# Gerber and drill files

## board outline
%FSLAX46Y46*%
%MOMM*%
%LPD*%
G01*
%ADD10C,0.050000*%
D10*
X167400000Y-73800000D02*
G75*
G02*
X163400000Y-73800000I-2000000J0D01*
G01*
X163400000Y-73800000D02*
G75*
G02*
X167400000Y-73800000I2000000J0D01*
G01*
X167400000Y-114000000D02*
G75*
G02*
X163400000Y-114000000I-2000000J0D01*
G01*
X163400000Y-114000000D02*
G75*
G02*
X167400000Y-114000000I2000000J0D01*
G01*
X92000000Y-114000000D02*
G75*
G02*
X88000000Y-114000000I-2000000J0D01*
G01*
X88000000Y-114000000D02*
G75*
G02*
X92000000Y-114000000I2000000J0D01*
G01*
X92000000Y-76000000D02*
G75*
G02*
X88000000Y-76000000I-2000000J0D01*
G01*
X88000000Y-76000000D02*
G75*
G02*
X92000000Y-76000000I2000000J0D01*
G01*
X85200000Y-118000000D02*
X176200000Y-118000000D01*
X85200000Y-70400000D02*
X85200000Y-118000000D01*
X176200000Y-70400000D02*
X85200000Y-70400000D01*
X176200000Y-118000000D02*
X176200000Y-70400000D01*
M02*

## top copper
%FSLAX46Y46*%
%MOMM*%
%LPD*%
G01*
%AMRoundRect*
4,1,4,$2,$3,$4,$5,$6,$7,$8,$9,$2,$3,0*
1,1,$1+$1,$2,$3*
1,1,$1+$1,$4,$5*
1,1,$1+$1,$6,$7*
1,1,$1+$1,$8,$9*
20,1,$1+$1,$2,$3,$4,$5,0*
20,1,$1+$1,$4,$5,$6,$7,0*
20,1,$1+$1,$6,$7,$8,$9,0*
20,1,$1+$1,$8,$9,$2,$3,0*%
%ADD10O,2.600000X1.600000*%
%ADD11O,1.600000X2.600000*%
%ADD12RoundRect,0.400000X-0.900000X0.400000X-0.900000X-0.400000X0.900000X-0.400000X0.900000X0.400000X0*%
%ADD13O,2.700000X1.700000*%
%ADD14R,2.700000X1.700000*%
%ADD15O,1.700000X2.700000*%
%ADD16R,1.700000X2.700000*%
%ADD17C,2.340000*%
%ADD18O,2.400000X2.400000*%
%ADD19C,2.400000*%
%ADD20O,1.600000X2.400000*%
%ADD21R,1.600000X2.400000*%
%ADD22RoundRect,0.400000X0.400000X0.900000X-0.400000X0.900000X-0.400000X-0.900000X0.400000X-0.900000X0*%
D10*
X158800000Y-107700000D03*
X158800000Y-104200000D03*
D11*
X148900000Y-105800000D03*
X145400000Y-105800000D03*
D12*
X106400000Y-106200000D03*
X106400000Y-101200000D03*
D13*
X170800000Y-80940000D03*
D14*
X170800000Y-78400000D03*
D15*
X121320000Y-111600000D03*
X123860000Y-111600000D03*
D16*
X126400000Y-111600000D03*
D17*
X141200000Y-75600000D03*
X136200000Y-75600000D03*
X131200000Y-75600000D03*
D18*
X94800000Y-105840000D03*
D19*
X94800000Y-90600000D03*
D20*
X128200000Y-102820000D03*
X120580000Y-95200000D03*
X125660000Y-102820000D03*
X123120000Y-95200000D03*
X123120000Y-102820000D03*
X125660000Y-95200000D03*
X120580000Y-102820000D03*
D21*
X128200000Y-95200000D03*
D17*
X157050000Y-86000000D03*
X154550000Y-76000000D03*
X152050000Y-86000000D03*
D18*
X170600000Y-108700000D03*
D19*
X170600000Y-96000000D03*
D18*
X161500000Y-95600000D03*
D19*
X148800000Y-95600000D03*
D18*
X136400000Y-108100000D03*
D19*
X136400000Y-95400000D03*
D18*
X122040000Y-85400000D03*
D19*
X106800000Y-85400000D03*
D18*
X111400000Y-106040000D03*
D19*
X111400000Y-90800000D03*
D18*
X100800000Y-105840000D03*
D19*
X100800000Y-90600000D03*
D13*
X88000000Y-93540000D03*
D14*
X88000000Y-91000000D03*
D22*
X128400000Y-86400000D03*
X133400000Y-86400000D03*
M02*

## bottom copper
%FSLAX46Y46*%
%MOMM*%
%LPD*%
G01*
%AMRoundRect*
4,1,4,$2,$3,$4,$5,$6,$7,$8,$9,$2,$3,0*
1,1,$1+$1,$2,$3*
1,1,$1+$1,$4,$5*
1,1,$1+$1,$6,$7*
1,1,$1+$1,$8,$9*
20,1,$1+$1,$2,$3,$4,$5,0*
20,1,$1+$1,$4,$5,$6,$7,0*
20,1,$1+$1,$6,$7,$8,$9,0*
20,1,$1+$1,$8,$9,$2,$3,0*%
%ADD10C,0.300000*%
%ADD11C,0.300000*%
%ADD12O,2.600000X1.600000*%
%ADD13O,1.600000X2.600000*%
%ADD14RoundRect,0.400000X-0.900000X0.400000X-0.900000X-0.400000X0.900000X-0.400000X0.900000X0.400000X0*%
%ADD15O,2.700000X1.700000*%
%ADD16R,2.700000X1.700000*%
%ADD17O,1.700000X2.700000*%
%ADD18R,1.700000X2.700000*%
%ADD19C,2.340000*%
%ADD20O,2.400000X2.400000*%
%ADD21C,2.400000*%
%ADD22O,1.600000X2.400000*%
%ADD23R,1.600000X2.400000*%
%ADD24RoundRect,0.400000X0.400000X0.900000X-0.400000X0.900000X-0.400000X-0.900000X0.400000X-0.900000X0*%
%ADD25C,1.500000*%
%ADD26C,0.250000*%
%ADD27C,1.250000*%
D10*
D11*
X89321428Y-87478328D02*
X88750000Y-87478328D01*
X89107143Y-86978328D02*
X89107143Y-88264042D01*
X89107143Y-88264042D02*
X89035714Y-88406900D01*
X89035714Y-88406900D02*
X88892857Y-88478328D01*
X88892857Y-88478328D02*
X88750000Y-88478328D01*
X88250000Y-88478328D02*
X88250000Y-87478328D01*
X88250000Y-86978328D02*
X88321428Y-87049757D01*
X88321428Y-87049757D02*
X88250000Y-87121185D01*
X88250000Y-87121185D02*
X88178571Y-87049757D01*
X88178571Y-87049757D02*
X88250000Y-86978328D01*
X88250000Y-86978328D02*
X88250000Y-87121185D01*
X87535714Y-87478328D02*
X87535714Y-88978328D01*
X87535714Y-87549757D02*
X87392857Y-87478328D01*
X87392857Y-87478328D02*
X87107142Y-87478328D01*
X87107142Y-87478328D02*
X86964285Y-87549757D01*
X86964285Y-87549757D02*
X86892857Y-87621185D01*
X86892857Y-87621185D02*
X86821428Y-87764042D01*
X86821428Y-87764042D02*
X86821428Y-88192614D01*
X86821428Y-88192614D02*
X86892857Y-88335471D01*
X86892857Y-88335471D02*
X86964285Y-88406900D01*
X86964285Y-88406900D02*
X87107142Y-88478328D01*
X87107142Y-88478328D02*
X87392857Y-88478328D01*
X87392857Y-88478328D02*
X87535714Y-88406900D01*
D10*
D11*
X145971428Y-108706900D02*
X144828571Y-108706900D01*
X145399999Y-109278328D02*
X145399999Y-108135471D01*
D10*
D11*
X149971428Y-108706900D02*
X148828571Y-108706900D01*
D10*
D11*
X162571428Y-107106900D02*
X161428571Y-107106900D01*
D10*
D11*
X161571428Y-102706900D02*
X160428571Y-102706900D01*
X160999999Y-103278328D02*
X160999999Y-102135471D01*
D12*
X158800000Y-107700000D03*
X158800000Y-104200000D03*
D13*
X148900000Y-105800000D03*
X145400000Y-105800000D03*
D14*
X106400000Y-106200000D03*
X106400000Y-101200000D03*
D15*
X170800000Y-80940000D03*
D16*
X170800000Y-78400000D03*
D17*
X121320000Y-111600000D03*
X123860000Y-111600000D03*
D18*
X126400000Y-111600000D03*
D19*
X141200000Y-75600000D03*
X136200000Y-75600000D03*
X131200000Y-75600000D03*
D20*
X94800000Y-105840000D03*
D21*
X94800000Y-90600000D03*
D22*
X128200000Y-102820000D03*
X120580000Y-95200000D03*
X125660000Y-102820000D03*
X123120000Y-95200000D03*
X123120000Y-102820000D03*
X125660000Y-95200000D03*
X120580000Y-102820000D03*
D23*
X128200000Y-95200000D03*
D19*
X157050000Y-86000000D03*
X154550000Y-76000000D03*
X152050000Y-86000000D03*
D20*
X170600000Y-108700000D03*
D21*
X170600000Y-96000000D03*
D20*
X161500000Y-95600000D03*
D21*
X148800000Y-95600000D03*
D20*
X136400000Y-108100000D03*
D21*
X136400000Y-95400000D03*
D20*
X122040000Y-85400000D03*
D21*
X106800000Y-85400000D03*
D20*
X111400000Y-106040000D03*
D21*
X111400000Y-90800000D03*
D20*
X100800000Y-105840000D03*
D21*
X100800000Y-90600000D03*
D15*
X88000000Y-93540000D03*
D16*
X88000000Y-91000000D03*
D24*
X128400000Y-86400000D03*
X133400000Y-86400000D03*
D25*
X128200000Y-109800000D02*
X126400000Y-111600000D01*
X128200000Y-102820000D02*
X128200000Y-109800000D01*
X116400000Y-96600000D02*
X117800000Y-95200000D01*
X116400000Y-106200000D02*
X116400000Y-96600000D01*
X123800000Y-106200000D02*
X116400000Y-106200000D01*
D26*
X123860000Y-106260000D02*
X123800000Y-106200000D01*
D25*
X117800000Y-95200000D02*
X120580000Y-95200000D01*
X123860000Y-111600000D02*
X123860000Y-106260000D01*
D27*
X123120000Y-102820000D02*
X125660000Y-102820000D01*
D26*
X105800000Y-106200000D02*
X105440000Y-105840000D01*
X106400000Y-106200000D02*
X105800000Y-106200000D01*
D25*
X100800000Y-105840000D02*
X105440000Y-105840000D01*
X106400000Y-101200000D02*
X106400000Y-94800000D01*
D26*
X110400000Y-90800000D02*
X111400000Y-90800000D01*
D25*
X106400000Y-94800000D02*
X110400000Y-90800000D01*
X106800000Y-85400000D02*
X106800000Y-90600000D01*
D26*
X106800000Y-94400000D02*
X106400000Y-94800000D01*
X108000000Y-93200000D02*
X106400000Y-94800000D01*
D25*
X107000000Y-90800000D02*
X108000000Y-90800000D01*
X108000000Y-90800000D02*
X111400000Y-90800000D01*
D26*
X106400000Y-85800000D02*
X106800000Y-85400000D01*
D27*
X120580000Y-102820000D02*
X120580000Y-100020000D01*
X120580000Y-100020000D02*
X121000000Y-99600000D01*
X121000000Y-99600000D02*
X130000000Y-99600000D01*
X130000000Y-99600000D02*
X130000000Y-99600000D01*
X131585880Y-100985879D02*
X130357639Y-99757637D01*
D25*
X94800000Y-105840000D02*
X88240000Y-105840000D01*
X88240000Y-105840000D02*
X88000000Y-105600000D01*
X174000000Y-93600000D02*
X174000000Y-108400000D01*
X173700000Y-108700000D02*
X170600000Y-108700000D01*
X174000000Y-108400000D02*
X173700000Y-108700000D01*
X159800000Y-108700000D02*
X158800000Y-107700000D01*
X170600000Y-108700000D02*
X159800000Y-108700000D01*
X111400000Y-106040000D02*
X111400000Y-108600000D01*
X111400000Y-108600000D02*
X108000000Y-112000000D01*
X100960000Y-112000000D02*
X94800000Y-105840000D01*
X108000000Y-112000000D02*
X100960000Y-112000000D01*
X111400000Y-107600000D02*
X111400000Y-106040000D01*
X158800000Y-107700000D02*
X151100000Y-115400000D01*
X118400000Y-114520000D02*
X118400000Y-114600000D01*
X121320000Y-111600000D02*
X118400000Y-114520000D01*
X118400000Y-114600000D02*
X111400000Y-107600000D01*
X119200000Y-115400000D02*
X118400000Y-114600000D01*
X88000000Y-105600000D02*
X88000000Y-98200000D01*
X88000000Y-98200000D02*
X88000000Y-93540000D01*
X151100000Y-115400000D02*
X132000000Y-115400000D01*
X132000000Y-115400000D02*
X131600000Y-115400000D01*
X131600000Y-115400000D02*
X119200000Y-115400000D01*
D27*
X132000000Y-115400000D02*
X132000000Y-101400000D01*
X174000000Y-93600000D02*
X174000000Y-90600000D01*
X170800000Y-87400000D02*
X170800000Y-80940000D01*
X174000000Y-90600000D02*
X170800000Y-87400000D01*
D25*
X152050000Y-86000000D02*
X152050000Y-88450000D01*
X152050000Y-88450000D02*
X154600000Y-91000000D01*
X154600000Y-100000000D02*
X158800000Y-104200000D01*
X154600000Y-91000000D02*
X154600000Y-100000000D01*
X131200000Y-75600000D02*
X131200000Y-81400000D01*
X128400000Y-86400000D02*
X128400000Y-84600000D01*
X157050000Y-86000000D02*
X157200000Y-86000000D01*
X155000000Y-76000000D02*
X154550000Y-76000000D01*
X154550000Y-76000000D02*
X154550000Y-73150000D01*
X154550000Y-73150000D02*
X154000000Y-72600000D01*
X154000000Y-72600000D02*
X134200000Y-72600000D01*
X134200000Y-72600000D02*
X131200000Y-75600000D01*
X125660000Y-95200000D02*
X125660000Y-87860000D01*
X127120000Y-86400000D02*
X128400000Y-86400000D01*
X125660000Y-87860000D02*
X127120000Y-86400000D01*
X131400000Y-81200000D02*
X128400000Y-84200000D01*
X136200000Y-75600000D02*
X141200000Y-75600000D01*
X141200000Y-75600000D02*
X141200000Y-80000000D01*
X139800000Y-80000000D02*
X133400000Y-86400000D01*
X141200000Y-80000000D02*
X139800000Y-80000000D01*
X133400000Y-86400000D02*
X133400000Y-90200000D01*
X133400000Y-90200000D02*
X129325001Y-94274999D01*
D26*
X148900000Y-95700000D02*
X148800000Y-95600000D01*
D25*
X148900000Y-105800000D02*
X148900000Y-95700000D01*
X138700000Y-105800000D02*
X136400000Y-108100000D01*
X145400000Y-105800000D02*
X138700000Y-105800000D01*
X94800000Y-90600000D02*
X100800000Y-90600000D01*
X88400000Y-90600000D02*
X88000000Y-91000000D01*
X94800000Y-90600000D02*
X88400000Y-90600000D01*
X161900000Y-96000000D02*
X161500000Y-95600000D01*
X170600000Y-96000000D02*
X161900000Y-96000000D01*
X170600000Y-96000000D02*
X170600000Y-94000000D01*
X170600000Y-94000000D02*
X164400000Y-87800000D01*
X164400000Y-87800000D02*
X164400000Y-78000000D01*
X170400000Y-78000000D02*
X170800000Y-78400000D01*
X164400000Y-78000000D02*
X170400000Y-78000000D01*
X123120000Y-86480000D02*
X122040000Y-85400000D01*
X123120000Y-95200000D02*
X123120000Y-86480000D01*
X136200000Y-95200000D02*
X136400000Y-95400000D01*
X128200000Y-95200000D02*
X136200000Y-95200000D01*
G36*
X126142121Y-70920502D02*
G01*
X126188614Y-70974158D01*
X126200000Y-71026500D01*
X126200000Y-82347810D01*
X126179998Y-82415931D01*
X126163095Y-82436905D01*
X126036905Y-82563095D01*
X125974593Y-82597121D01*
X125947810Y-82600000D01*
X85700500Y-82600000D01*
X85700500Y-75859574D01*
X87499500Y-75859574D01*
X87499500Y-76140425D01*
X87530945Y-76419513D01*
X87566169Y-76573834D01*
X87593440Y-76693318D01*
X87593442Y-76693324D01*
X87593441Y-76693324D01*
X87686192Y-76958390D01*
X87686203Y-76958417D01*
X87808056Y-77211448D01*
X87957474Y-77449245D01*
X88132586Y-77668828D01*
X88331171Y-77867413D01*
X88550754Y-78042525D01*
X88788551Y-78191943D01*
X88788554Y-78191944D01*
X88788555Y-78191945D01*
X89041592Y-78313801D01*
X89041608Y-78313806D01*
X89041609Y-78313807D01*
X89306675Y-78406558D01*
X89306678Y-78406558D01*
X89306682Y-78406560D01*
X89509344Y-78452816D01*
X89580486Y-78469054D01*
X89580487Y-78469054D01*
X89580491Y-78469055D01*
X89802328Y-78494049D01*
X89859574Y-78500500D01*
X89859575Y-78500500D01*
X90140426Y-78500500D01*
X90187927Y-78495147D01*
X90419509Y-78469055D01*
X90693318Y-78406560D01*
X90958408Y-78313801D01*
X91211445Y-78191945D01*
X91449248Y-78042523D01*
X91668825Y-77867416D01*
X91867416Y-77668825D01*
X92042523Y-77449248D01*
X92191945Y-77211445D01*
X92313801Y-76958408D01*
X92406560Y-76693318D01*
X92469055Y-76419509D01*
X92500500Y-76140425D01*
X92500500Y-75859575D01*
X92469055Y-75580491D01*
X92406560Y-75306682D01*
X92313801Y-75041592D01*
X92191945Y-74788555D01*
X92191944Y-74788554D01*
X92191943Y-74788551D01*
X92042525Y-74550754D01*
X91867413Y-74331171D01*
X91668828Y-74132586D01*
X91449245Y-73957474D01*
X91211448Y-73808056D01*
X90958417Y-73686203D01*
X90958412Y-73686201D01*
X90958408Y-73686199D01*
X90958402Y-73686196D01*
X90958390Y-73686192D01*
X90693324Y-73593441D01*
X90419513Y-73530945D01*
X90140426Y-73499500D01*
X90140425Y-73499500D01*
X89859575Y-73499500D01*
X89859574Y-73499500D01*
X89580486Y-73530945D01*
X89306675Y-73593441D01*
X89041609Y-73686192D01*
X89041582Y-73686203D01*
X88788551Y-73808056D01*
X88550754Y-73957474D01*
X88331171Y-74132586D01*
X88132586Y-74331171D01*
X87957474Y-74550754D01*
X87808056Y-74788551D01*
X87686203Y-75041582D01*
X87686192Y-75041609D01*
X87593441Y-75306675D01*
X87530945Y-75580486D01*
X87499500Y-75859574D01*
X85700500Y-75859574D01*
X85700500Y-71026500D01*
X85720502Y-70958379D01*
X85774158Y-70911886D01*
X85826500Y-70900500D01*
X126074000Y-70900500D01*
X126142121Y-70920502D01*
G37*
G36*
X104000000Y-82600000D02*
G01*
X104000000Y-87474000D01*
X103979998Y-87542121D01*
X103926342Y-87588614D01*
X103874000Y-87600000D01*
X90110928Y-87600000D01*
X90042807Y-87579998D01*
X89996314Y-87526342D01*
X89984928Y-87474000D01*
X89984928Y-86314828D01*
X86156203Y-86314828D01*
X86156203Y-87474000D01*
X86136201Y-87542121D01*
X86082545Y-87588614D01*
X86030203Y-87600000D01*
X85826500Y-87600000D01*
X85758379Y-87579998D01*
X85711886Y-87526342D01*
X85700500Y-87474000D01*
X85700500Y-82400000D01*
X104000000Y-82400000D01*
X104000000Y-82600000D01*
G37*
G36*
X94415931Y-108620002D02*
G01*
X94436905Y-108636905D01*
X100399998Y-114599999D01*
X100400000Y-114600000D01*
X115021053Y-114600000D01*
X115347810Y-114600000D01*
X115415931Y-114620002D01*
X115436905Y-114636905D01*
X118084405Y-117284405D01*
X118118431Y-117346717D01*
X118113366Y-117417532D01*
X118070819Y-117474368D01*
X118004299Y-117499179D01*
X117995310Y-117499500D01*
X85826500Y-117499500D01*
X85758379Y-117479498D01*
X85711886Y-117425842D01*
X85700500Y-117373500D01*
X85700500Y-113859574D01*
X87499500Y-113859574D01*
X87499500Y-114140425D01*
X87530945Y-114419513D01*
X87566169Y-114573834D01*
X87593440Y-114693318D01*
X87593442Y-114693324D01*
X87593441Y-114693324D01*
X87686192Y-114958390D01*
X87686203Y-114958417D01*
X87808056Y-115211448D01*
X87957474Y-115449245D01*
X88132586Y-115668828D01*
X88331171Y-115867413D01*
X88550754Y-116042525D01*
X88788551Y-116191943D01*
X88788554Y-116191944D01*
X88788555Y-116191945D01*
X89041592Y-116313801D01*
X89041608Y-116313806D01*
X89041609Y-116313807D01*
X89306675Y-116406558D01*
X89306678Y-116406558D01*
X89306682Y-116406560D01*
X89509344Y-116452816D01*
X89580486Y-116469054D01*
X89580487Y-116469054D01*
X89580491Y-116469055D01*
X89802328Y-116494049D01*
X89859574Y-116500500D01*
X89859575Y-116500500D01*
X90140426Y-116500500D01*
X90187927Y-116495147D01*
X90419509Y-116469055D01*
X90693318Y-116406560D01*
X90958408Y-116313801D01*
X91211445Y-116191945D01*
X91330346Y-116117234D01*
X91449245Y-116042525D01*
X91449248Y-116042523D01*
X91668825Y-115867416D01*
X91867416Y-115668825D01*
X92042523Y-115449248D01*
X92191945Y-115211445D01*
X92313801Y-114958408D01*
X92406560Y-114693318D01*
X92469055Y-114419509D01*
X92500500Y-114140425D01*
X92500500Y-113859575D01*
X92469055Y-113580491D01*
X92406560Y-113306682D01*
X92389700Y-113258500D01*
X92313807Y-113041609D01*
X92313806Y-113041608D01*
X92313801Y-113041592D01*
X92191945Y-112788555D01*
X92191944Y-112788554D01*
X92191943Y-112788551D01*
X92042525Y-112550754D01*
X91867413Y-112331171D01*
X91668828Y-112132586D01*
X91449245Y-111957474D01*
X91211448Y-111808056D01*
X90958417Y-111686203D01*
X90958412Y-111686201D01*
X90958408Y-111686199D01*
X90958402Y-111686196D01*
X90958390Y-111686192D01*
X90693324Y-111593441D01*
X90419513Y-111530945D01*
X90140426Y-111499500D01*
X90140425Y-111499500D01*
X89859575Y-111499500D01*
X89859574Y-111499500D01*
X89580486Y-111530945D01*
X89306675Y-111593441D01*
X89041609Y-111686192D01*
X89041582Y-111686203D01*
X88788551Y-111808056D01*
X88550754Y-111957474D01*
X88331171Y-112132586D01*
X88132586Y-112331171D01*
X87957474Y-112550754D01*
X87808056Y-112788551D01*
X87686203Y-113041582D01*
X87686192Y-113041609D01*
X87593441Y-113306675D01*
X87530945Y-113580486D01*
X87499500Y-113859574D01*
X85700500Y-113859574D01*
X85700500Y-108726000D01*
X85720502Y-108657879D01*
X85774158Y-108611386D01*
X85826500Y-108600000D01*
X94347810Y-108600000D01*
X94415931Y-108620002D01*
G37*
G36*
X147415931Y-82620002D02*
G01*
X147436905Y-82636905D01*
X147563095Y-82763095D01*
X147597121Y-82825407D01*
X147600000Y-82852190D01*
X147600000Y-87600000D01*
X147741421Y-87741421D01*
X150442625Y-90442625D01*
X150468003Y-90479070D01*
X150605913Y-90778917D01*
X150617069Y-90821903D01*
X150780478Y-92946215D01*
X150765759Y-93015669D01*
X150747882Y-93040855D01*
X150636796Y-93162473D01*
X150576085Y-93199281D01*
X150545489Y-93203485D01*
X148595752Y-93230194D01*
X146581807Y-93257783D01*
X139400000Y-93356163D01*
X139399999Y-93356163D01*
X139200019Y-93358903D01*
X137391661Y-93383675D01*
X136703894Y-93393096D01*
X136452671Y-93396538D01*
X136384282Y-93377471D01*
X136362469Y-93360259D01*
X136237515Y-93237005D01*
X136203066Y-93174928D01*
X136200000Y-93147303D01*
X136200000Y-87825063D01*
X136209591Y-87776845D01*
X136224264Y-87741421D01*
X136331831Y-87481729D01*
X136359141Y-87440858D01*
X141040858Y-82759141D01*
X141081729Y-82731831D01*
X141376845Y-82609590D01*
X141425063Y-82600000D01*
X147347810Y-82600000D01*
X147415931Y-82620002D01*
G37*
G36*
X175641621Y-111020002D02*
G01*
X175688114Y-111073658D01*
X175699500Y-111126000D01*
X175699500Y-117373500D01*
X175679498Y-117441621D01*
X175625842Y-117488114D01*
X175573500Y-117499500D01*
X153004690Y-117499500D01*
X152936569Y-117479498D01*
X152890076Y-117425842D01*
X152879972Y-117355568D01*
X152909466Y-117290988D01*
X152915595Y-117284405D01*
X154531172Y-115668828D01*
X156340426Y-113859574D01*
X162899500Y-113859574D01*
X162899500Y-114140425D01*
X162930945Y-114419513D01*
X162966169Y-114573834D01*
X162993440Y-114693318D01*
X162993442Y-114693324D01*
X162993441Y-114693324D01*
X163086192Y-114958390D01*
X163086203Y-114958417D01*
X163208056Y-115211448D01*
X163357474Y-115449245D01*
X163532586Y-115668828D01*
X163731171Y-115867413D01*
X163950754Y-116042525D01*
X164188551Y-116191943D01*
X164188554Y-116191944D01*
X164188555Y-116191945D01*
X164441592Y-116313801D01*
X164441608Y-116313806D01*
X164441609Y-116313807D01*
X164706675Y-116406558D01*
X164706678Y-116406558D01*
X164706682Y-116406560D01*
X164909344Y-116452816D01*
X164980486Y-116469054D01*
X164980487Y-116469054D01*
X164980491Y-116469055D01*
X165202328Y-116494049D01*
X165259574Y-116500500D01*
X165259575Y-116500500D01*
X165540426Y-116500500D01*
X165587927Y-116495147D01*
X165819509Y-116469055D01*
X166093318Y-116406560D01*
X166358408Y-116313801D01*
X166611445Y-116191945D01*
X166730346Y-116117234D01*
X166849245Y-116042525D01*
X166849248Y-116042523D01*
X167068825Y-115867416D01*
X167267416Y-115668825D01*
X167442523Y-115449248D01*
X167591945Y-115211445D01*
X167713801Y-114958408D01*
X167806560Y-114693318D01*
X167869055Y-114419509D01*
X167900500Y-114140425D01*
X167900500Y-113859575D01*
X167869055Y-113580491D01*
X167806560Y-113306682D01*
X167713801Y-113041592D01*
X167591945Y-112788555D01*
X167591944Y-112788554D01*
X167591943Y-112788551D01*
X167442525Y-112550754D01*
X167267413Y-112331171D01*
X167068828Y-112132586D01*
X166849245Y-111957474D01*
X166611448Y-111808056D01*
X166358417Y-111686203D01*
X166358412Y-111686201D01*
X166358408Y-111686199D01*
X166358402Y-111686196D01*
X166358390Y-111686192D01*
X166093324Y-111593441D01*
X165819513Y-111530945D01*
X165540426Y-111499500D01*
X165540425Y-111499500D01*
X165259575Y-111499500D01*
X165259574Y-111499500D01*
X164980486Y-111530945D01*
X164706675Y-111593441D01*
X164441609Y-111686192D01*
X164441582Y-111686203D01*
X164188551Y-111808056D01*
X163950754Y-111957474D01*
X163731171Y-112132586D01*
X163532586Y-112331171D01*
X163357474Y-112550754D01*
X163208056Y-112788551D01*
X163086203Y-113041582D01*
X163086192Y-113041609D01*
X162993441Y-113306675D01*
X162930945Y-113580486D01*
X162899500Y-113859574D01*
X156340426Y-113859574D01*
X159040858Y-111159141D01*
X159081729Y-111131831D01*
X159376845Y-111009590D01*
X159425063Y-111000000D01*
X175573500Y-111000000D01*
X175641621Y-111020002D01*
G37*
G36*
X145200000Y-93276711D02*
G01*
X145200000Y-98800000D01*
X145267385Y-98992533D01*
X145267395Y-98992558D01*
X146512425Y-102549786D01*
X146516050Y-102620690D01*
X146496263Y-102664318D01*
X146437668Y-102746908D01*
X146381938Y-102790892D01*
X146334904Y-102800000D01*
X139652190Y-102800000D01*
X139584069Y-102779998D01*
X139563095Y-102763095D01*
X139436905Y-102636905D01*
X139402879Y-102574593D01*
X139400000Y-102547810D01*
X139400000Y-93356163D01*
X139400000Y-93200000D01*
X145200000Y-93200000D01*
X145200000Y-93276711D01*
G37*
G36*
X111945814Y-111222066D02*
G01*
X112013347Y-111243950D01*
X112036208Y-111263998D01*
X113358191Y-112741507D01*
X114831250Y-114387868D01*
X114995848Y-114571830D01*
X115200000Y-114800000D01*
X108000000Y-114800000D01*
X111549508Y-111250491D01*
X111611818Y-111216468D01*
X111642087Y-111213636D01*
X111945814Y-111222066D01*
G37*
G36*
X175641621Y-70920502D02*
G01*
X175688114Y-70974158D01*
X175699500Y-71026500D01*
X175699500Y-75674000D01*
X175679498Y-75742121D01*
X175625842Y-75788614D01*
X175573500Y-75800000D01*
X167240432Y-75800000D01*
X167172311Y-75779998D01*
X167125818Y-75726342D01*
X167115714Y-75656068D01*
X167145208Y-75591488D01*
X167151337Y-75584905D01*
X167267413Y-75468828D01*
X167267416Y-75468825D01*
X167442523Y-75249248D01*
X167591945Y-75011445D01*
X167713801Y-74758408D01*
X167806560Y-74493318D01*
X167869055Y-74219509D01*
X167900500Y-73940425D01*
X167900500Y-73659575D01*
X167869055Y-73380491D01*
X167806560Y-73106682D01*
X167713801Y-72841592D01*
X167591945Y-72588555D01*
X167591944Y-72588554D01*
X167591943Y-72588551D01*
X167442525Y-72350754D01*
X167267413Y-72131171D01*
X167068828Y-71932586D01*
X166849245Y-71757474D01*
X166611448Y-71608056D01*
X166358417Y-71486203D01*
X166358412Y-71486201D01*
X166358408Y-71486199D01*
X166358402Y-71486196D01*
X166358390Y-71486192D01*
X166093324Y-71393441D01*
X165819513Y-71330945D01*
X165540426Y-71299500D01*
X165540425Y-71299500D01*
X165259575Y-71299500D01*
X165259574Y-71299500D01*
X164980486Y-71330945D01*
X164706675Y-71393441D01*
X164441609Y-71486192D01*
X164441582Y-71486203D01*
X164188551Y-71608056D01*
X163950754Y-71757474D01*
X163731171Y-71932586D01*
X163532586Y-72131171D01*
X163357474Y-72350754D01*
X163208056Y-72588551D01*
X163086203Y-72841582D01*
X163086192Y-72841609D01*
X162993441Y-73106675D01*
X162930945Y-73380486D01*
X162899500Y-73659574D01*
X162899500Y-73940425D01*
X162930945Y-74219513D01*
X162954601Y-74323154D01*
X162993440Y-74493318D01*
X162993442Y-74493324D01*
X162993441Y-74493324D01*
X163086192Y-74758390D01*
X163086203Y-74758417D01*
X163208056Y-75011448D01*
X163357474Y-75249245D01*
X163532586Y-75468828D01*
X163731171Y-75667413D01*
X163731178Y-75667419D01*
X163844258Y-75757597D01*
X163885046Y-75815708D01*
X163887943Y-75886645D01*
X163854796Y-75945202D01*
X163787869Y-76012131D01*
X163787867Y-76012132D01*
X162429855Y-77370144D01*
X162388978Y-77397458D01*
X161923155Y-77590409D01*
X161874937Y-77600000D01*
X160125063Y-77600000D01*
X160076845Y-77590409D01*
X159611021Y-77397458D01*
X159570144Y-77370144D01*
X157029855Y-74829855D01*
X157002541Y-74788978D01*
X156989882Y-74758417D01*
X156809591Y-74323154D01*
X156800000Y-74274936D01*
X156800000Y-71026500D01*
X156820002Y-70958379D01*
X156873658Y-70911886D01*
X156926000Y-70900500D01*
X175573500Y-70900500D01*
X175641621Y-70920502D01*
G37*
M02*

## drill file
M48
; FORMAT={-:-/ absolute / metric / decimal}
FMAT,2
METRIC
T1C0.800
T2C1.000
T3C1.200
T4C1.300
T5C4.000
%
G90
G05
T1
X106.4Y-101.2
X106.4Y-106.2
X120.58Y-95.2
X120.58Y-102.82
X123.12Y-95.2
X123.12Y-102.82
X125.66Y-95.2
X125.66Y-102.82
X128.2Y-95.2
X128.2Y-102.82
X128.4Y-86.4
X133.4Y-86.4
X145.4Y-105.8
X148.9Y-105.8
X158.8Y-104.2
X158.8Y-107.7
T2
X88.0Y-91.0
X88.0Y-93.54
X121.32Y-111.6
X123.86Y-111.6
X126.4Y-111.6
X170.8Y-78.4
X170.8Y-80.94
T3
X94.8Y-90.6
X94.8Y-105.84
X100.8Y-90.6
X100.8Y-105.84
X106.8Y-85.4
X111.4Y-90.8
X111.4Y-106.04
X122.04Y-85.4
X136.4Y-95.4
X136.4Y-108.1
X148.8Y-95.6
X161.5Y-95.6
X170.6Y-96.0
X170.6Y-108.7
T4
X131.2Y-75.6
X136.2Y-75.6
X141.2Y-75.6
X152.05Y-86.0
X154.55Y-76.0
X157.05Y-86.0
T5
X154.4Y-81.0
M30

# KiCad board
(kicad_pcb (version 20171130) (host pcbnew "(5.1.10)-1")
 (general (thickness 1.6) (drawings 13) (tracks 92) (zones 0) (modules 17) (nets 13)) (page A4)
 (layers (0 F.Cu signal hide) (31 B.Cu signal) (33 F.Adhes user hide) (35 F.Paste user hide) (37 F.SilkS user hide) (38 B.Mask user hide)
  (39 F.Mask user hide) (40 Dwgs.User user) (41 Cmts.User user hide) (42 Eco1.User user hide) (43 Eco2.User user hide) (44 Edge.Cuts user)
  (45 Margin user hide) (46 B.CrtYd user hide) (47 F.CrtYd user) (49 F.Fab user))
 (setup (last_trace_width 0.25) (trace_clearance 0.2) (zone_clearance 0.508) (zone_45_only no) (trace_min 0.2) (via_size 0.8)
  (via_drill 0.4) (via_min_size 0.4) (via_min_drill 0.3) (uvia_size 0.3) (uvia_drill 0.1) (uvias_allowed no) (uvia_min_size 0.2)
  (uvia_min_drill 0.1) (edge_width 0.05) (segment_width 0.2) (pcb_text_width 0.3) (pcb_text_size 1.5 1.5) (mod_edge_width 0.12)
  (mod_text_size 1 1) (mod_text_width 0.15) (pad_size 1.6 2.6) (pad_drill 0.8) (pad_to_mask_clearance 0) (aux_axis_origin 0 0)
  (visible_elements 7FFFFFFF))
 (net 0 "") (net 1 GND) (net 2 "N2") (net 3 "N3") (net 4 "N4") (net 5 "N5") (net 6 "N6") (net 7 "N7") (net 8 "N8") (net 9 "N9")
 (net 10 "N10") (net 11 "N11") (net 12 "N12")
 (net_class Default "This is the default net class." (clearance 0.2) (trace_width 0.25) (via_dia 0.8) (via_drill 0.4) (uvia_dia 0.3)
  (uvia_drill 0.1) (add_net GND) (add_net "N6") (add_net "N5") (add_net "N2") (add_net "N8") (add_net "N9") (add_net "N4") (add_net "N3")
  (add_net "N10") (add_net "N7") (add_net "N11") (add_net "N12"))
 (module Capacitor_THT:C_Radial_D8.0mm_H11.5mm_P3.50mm (layer F.Cu) (at 158.8 104.2 270)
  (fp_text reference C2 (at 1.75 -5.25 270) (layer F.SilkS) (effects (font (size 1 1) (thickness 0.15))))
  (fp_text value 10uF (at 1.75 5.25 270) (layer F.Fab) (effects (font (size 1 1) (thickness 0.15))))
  (pad 2 thru_hole oval (at 3.5 0 270) (size 1.6 2.6) (drill 0.8) (layers *.Cu *.Mask) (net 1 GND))
  (pad 1 thru_hole oval (at 0 0 270) (size 1.6 2.6) (drill 0.8) (layers *.Cu *.Mask) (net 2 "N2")))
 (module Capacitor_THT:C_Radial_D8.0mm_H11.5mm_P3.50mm (layer F.Cu) (at 145.4 105.8)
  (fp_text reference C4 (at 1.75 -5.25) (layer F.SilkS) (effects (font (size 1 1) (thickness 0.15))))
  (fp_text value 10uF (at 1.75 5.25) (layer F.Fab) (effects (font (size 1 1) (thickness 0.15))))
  (pad 2 thru_hole oval (at 3.5 0) (size 1.6 2.6) (drill 0.8) (layers *.Cu *.Mask) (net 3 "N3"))
  (pad 1 thru_hole oval (at 0 0) (size 1.6 2.6) (drill 0.8) (layers *.Cu *.Mask) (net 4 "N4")))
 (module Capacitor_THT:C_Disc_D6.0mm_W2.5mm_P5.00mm (layer F.Cu) (at 106.4 101.2 270)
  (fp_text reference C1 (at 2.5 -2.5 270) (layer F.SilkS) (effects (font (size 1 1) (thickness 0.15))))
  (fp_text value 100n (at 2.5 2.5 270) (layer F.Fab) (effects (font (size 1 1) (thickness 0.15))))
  (pad 2 thru_hole roundrect (at 5 0 270) (size 1.6 2.6) (drill 0.8) (layers *.Cu *.Mask) (roundrect_rratio 0.25) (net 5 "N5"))
  (pad 1 thru_hole roundrect (at 0 0 270) (size 1.6 2.6) (drill 0.8) (layers *.Cu *.Mask) (roundrect_rratio 0.25) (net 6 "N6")))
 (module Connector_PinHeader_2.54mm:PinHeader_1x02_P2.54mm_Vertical (layer F.Cu) (at 170.8 78.4)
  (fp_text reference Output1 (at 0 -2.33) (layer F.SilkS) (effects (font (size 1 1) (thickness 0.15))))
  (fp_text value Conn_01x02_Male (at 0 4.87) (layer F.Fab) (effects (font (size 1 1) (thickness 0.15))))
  (pad 2 thru_hole oval (at 0 2.54) (size 2.7 1.7) (drill 1) (layers *.Cu *.Mask) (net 1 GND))
  (pad 1 thru_hole rect (at 0 0) (size 2.7 1.7) (drill 1) (layers *.Cu *.Mask) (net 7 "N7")))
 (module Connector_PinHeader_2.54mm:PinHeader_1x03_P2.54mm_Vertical (layer F.Cu) (at 126.4 111.6 270)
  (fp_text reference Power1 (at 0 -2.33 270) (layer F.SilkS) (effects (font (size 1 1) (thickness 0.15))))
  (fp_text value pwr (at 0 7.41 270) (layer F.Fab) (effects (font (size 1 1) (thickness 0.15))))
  (pad 3 thru_hole oval (at 0 5.08 270) (size 2.7 1.7) (drill 1) (layers *.Cu *.Mask) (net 1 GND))
  (pad 2 thru_hole oval (at 0 2.54 270) (size 2.7 1.7) (drill 1) (layers *.Cu *.Mask))
  (pad 1 thru_hole rect (at 0 0 270) (size 2.7 1.7) (drill 1) (layers *.Cu *.Mask)))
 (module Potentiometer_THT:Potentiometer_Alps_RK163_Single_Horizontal (layer F.Cu) (at 141.2 75.6 90)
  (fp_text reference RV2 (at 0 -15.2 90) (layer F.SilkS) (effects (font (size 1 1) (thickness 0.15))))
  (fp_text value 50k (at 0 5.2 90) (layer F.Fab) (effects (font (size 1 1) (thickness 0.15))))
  (pad 1 thru_hole circle (at 0 0 90) (size 2.34 2.34) (drill 1.3) (layers *.Cu *.Mask) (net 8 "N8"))
  (pad 2 thru_hole circle (at 0 -5 90) (size 2.34 2.34) (drill 1.3) (layers *.Cu *.Mask) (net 8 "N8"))
  (pad 3 thru_hole circle (at 0 -10 90) (size 2.34 2.34) (drill 1.3) (layers *.Cu *.Mask) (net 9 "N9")))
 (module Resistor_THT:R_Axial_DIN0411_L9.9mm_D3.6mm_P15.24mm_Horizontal (layer F.Cu) (at 94.8 90.6 270)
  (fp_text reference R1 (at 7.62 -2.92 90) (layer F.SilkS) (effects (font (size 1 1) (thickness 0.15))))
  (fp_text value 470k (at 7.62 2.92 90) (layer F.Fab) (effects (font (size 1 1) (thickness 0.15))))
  (pad 2 thru_hole oval (at 15.24 0 270) (size 2.4 2.4) (drill 1.2) (layers *.Cu *.Mask) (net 1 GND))
  (pad 1 thru_hole circle (at 0 0 270) (size 2.4 2.4) (drill 1.2) (layers *.Cu *.Mask) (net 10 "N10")))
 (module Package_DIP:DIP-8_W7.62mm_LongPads (layer F.Cu) (at 128.2 95.2 270)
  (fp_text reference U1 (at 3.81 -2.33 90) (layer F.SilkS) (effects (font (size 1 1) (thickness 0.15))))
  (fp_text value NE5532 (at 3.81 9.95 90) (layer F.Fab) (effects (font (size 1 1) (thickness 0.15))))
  (pad 8 thru_hole oval (at 7.62 0 270) (size 2.4 1.6) (drill 0.8) (layers *.Cu *.Mask))
  (pad 4 thru_hole oval (at 0 7.62 270) (size 2.4 1.6) (drill 0.8) (layers *.Cu *.Mask))
  (pad 7 thru_hole oval (at 7.62 2.54 270) (size 2.4 1.6) (drill 0.8) (layers *.Cu *.Mask))
  (pad 3 thru_hole oval (at 0 5.08 270) (size 2.4 1.6) (drill 0.8) (layers *.Cu *.Mask) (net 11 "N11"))
  (pad 6 thru_hole oval (at 7.62 5.08 270) (size 2.4 1.6) (drill 0.8) (layers *.Cu *.Mask))
  (pad 2 thru_hole oval (at 0 2.54 270) (size 2.4 1.6) (drill 0.8) (layers *.Cu *.Mask) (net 9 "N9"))
  (pad 5 thru_hole oval (at 7.62 7.62 270) (size 2.4 1.6) (drill 0.8) (layers *.Cu *.Mask) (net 1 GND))
  (pad 1 thru_hole rect (at 0 0 270) (size 2.4 1.6) (drill 0.8) (layers *.Cu *.Mask) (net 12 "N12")))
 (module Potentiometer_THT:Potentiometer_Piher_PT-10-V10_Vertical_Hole (layer F.Cu) (at 157.05 86 90)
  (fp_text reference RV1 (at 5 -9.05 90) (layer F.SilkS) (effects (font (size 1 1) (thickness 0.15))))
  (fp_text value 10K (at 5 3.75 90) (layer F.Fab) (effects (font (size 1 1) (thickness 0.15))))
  (pad "" np_thru_hole circle (at 5 -2.65 90) (size 4 4) (drill 4) (layers *.Cu *.Mask))
  (pad 1 thru_hole circle (at 0 0 90) (size 2.34 2.34) (drill 1.3) (layers *.Cu *.Mask) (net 9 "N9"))
  (pad 2 thru_hole circle (at 10 -2.5 90) (size 2.34 2.34) (drill 1.3) (layers *.Cu *.Mask) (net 9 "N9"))
  (pad 3 thru_hole circle (at 0 -5 90) (size 2.34 2.34) (drill 1.3) (layers *.Cu *.Mask) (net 2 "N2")))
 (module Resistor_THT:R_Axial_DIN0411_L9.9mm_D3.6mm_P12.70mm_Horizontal (layer F.Cu) (at 170.6 96 270)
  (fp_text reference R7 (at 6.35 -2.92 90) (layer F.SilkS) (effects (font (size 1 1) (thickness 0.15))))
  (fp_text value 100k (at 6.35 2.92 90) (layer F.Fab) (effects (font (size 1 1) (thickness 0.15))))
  (pad 2 thru_hole oval (at 12.7 0 270) (size 2.4 2.4) (drill 1.2) (layers *.Cu *.Mask) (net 1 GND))
  (pad 1 thru_hole circle (at 0 0 270) (size 2.4 2.4) (drill 1.2) (layers *.Cu *.Mask) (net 7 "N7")))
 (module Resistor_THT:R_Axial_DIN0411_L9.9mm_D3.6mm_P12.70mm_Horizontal (layer F.Cu) (at 148.8 95.6)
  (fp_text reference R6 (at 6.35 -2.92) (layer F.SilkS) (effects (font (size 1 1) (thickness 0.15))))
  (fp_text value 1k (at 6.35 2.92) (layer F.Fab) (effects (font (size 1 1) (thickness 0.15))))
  (pad 2 thru_hole oval (at 12.7 0) (size 2.4 2.4) (drill 1.2) (layers *.Cu *.Mask) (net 7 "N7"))
  (pad 1 thru_hole circle (at 0 0) (size 2.4 2.4) (drill 1.2) (layers *.Cu *.Mask) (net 3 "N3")))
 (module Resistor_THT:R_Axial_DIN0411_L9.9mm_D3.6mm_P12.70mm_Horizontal (layer F.Cu) (at 136.4 95.4 270)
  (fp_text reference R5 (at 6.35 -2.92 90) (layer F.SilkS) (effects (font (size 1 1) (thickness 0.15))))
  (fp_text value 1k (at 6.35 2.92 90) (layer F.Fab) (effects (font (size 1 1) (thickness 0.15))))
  (pad 2 thru_hole oval (at 12.7 0 270) (size 2.4 2.4) (drill 1.2) (layers *.Cu *.Mask) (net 4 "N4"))
  (pad 1 thru_hole circle (at 0 0 270) (size 2.4 2.4) (drill 1.2) (layers *.Cu *.Mask) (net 12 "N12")))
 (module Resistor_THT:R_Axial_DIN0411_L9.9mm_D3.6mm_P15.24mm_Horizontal (layer F.Cu) (at 106.8 85.4)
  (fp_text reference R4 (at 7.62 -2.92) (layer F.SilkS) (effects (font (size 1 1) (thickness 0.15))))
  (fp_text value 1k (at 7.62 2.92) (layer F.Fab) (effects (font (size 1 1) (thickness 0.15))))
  (pad 2 thru_hole oval (at 15.24 0) (size 2.4 2.4) (drill 1.2) (layers *.Cu *.Mask) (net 11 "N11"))
  (pad 1 thru_hole circle (at 0 0) (size 2.4 2.4) (drill 1.2) (layers *.Cu *.Mask) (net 6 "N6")))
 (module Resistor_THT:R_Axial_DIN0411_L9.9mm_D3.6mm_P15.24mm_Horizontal (layer F.Cu) (at 111.4 90.8 270)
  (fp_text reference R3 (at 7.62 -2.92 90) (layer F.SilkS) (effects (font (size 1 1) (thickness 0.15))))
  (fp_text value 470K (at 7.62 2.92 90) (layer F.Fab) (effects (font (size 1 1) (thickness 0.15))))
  (pad 2 thru_hole oval (at 15.24 0 270) (size 2.4 2.4) (drill 1.2) (layers *.Cu *.Mask) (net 1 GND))
  (pad 1 thru_hole circle (at 0 0 270) (size 2.4 2.4) (drill 1.2) (layers *.Cu *.Mask) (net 6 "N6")))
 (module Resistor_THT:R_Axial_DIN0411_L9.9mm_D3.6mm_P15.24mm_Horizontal (layer F.Cu) (at 100.8 90.6 270)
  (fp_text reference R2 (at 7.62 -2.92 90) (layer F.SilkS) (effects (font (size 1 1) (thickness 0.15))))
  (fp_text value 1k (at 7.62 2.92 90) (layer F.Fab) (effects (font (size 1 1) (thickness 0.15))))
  (pad 2 thru_hole oval (at 15.24 0 270) (size 2.4 2.4) (drill 1.2) (layers *.Cu *.Mask) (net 5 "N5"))
  (pad 1 thru_hole circle (at 0 0 270) (size 2.4 2.4) (drill 1.2) (layers *.Cu *.Mask) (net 10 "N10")))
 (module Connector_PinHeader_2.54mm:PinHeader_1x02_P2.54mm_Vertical (layer F.Cu) (at 88 91)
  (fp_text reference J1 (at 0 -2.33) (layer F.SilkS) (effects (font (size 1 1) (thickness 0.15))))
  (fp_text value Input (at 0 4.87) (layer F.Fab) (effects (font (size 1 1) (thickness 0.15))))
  (pad 2 thru_hole oval (at 0 2.54) (size 2.7 1.7) (drill 1) (layers *.Cu *.Mask) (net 1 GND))
  (pad 1 thru_hole rect (at 0 0) (size 2.7 1.7) (drill 1) (layers *.Cu *.Mask) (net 10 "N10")))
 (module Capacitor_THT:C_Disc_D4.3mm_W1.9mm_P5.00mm (layer F.Cu) (at 133.4 86.4 180)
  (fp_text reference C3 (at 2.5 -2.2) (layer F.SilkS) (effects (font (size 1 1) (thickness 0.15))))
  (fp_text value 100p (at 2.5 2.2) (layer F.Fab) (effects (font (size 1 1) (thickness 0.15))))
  (pad 2 thru_hole roundrect (at 5 0 180) (size 1.6 2.6) (drill 0.8) (layers *.Cu *.Mask) (roundrect_rratio 0.25) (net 9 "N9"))
  (pad 1 thru_hole roundrect (at 0 0 180) (size 1.6 2.6) (drill 0.8) (layers *.Cu *.Mask) (roundrect_rratio 0.25) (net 8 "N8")))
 (gr_circle (center 165.4 73.8) (end 163.8 72.6) (layer Edge.Cuts) (width 0.05))
 (gr_circle (center 165.4 114) (end 163.8 112.8) (layer Edge.Cuts) (width 0.05))
 (gr_circle (center 90 114) (end 88.4 112.8) (layer Edge.Cuts) (width 0.05))
 (gr_circle (center 90 76) (end 88.4 74.8) (layer Edge.Cuts) (width 0.05))
 (gr_line (start 85.2 118) (end 176.2 118) (layer Edge.Cuts) (width 0.05))
 (gr_line (start 85.2 70.4) (end 85.2 118) (layer Edge.Cuts) (width 0.05))
 (gr_line (start 176.2 70.4) (end 85.2 70.4) (layer Edge.Cuts) (width 0.05))
 (gr_line (start 176.2 118) (end 176.2 70.4) (layer Edge.Cuts) (width 0.05))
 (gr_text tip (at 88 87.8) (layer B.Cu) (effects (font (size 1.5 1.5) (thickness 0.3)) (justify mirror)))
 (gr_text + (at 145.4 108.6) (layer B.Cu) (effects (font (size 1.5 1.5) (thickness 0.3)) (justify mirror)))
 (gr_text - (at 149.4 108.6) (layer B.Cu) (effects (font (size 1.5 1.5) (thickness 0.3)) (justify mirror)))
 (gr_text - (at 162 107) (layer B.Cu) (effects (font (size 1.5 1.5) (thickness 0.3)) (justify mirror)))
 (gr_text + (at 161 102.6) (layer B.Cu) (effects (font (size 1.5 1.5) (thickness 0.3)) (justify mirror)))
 (segment (start 128.2 109.8) (end 126.4 111.6) (width 1.5) (layer B.Cu) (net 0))
 (segment (start 128.2 102.82) (end 128.2 109.8) (width 1.5) (layer B.Cu) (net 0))
 (segment (start 116.4 96.6) (end 117.8 95.2) (width 1.5) (layer B.Cu) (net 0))
 (segment (start 116.4 106.2) (end 116.4 96.6) (width 1.5) (layer B.Cu) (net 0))
 (segment (start 123.8 106.2) (end 116.4 106.2) (width 1.5) (layer B.Cu) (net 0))
 (segment (start 123.86 106.26) (end 123.8 106.2) (width 0.25) (layer B.Cu) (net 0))
 (segment (start 117.8 95.2) (end 120.58 95.2) (width 1.5) (layer B.Cu) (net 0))
 (segment (start 123.86 111.6) (end 123.86 106.26) (width 1.5) (layer B.Cu) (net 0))
 (segment (start 123.12 102.82) (end 125.66 102.82) (width 1.25) (layer B.Cu) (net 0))
 (segment (start 105.8 106.2) (end 105.44 105.84) (width 0.25) (layer B.Cu) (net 5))
 (segment (start 106.4 106.2) (end 105.8 106.2) (width 0.25) (layer B.Cu) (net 5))
 (segment (start 100.8 105.84) (end 105.44 105.84) (width 1.5) (layer B.Cu) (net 5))
 (segment (start 106.4 101.2) (end 106.4 94.8) (width 1.5) (layer B.Cu) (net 6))
 (segment (start 110.4 90.8) (end 111.4 90.8) (width 0.25) (layer B.Cu) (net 6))
 (segment (start 106.4 94.8) (end 110.4 90.8) (width 1.5) (layer B.Cu) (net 6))
 (segment (start 106.8 85.4) (end 106.8 90.6) (width 1.5) (layer B.Cu) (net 6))
 (segment (start 106.8 94.4) (end 106.4 94.8) (width 0.25) (layer B.Cu) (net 6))
 (segment (start 108 93.2) (end 106.4 94.8) (width 0.25) (layer B.Cu) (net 6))
 (segment (start 107 90.8) (end 108 90.8) (width 1.5) (layer B.Cu) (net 6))
 (segment (start 108 90.8) (end 111.4 90.8) (width 1.5) (layer B.Cu) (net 6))
 (segment (start 106.4 85.8) (end 106.8 85.4) (width 0.25) (layer B.Cu) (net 6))
 (segment (start 120.58 102.82) (end 120.58 100.02) (width 1.25) (layer B.Cu) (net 1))
 (segment (start 120.58 100.02) (end 121 99.6) (width 1.25) (layer B.Cu) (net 1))
 (segment (start 121 99.6) (end 130 99.6) (width 1.25) (layer B.Cu) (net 1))
 (segment (start 130 99.6) (end 130 99.6) (width 1.25) (layer B.Cu) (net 1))
 (segment (start 131.58588 100.985879) (end 130.357639 99.757637) (width 1.25) (layer B.Cu) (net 1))
 (segment (start 94.8 105.84) (end 88.24 105.84) (width 1.5) (layer B.Cu) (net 1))
 (segment (start 88.24 105.84) (end 88 105.6) (width 1.5) (layer B.Cu) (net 1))
 (segment (start 174 93.6) (end 174 108.4) (width 1.5) (layer B.Cu) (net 1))
 (segment (start 173.7 108.7) (end 170.6 108.7) (width 1.5) (layer B.Cu) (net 1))
 (segment (start 174 108.4) (end 173.7 108.7) (width 1.5) (layer B.Cu) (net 1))
 (segment (start 159.8 108.7) (end 158.8 107.7) (width 1.5) (layer B.Cu) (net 1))
 (segment (start 170.6 108.7) (end 159.8 108.7) (width 1.5) (layer B.Cu) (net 1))
 (segment (start 111.4 106.04) (end 111.4 108.6) (width 1.5) (layer B.Cu) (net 1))
 (segment (start 111.4 108.6) (end 108 112) (width 1.5) (layer B.Cu) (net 1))
 (segment (start 100.96 112) (end 94.8 105.84) (width 1.5) (layer B.Cu) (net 1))
 (segment (start 108 112) (end 100.96 112) (width 1.5) (layer B.Cu) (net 1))
 (segment (start 111.4 107.6) (end 111.4 106.04) (width 1.5) (layer B.Cu) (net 1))
 (segment (start 158.8 107.7) (end 151.1 115.4) (width 1.5) (layer B.Cu) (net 1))
 (segment (start 118.4 114.52) (end 118.4 114.6) (width 1.5) (layer B.Cu) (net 1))
 (segment (start 121.32 111.6) (end 118.4 114.52) (width 1.5) (layer B.Cu) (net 1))
 (segment (start 118.4 114.6) (end 111.4 107.6) (width 1.5) (layer B.Cu) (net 1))
 (segment (start 119.2 115.4) (end 118.4 114.6) (width 1.5) (layer B.Cu) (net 1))
 (segment (start 88 105.6) (end 88 98.2) (width 1.5) (layer B.Cu) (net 1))
 (segment (start 88 98.2) (end 88 93.54) (width 1.5) (layer B.Cu) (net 1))
 (segment (start 151.1 115.4) (end 132 115.4) (width 1.5) (layer B.Cu) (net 1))
 (segment (start 132 115.4) (end 131.6 115.4) (width 1.5) (layer B.Cu) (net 1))
 (segment (start 131.6 115.4) (end 119.2 115.4) (width 1.5) (layer B.Cu) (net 1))
 (segment (start 132 115.4) (end 132 101.4) (width 1.25) (layer B.Cu) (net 1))
 (segment (start 174 93.6) (end 174 90.6) (width 1.25) (layer B.Cu) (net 1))
 (segment (start 170.8 87.4) (end 170.8 80.94) (width 1.25) (layer B.Cu) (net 1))
 (segment (start 174 90.6) (end 170.8 87.4) (width 1.25) (layer B.Cu) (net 1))
 (segment (start 152.05 86) (end 152.05 88.45) (width 1.5) (layer B.Cu) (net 2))
 (segment (start 152.05 88.45) (end 154.6 91) (width 1.5) (layer B.Cu) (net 2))
 (segment (start 154.6 100) (end 158.8 104.2) (width 1.5) (layer B.Cu) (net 2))
 (segment (start 154.6 91) (end 154.6 100) (width 1.5) (layer B.Cu) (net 2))
 (segment (start 131.2 75.6) (end 131.2 81.4) (width 1.5) (layer B.Cu) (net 9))
 (segment (start 128.4 86.4) (end 128.4 84.6) (width 1.5) (layer B.Cu) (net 9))
 (segment (start 157.05 86) (end 157.2 86) (width 1.5) (layer B.Cu) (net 9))
 (segment (start 155 76) (end 154.55 76) (width 1.5) (layer B.Cu) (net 9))
 (segment (start 154.55 76) (end 154.55 73.15) (width 1.5) (layer B.Cu) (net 9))
 (segment (start 154.55 73.15) (end 154 72.6) (width 1.5) (layer B.Cu) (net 9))
 (segment (start 154 72.6) (end 134.2 72.6) (width 1.5) (layer B.Cu) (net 9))
 (segment (start 134.2 72.6) (end 131.2 75.6) (width 1.5) (layer B.Cu) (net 9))
 (segment (start 125.66 95.2) (end 125.66 87.86) (width 1.5) (layer B.Cu) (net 9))
 (segment (start 127.12 86.4) (end 128.4 86.4) (width 1.5) (layer B.Cu) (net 9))
 (segment (start 125.66 87.86) (end 127.12 86.4) (width 1.5) (layer B.Cu) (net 9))
 (segment (start 131.4 81.2) (end 128.4 84.2) (width 1.5) (layer B.Cu) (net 9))
 (segment (start 136.2 75.6) (end 141.2 75.6) (width 1.5) (layer B.Cu) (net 8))
 (segment (start 141.2 75.6) (end 141.2 80) (width 1.5) (layer B.Cu) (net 8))
 (segment (start 139.8 80) (end 133.4 86.4) (width 1.5) (layer B.Cu) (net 8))
 (segment (start 141.2 80) (end 139.8 80) (width 1.5) (layer B.Cu) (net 8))
 (segment (start 133.4 86.4) (end 133.4 90.2) (width 1.5) (layer B.Cu) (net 8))
 (segment (start 133.4 90.2) (end 129.325001 94.274999) (width 1.5) (layer B.Cu) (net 8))
 (segment (start 148.9 95.7) (end 148.8 95.6) (width 0.25) (layer B.Cu) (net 3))
 (segment (start 148.9 105.8) (end 148.9 95.7) (width 1.5) (layer B.Cu) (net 3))
 (segment (start 138.7 105.8) (end 136.4 108.1) (width 1.5) (layer B.Cu) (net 4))
 (segment (start 145.4 105.8) (end 138.7 105.8) (width 1.5) (layer B.Cu) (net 4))
 (segment (start 94.8 90.6) (end 100.8 90.6) (width 1.5) (layer B.Cu) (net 10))
 (segment (start 88.4 90.6) (end 88 91) (width 1.5) (layer B.Cu) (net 10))
 (segment (start 94.8 90.6) (end 88.4 90.6) (width 1.5) (layer B.Cu) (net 10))
 (segment (start 161.9 96) (end 161.5 95.6) (width 1.5) (layer B.Cu) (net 7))
 (segment (start 170.6 96) (end 161.9 96) (width 1.5) (layer B.Cu) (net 7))
 (segment (start 170.6 96) (end 170.6 94) (width 1.5) (layer B.Cu) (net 7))
 (segment (start 170.6 94) (end 164.4 87.8) (width 1.5) (layer B.Cu) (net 7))
 (segment (start 164.4 87.8) (end 164.4 78) (width 1.5) (layer B.Cu) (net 7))
 (segment (start 170.4 78) (end 170.8 78.4) (width 1.5) (layer B.Cu) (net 7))
 (segment (start 164.4 78) (end 170.4 78) (width 1.5) (layer B.Cu) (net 7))
 (segment (start 123.12 86.48) (end 122.04 85.4) (width 1.5) (layer B.Cu) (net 11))
 (segment (start 123.12 95.2) (end 123.12 86.48) (width 1.5) (layer B.Cu) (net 11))
 (segment (start 136.2 95.2) (end 136.4 95.4) (width 1.5) (layer B.Cu) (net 12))
 (segment (start 128.2 95.2) (end 136.2 95.2) (width 1.5) (layer B.Cu) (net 12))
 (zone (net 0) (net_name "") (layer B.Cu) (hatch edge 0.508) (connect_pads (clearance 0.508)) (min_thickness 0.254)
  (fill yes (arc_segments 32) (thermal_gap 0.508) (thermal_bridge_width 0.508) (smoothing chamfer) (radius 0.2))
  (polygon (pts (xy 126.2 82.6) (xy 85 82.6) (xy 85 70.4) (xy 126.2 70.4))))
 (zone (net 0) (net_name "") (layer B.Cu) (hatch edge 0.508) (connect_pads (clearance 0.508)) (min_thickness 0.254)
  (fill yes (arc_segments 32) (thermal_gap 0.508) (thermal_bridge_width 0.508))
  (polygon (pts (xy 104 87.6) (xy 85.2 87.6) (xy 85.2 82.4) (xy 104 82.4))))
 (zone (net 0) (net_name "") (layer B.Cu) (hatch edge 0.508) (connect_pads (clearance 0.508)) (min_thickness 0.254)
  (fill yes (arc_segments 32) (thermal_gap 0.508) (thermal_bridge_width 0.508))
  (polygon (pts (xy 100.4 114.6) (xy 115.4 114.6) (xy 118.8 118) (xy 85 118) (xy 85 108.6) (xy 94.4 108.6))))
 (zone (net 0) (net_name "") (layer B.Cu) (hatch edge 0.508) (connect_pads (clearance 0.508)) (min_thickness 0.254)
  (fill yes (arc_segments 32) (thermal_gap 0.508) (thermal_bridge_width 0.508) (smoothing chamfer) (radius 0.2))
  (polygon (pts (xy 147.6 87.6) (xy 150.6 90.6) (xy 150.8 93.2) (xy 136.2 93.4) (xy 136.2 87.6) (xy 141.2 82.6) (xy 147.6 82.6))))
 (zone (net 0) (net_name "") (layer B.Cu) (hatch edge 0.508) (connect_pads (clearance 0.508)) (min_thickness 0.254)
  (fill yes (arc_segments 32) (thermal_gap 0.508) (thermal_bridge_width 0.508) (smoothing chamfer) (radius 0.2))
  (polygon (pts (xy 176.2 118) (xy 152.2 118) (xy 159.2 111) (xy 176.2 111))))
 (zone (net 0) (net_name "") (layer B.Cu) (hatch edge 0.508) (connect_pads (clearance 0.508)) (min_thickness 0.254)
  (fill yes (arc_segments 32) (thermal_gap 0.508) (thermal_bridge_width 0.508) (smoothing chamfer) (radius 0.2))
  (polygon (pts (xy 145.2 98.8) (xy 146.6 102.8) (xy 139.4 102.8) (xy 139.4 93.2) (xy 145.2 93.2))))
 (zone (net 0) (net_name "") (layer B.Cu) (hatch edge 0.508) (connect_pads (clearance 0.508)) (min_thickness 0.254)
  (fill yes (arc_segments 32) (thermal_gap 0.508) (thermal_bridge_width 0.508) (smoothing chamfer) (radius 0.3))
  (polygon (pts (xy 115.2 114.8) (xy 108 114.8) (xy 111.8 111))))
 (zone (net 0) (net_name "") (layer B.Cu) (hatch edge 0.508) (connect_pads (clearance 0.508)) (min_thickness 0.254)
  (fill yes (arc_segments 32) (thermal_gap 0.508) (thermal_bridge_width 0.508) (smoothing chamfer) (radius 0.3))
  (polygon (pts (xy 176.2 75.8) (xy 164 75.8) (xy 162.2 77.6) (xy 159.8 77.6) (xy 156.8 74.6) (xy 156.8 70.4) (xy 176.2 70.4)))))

